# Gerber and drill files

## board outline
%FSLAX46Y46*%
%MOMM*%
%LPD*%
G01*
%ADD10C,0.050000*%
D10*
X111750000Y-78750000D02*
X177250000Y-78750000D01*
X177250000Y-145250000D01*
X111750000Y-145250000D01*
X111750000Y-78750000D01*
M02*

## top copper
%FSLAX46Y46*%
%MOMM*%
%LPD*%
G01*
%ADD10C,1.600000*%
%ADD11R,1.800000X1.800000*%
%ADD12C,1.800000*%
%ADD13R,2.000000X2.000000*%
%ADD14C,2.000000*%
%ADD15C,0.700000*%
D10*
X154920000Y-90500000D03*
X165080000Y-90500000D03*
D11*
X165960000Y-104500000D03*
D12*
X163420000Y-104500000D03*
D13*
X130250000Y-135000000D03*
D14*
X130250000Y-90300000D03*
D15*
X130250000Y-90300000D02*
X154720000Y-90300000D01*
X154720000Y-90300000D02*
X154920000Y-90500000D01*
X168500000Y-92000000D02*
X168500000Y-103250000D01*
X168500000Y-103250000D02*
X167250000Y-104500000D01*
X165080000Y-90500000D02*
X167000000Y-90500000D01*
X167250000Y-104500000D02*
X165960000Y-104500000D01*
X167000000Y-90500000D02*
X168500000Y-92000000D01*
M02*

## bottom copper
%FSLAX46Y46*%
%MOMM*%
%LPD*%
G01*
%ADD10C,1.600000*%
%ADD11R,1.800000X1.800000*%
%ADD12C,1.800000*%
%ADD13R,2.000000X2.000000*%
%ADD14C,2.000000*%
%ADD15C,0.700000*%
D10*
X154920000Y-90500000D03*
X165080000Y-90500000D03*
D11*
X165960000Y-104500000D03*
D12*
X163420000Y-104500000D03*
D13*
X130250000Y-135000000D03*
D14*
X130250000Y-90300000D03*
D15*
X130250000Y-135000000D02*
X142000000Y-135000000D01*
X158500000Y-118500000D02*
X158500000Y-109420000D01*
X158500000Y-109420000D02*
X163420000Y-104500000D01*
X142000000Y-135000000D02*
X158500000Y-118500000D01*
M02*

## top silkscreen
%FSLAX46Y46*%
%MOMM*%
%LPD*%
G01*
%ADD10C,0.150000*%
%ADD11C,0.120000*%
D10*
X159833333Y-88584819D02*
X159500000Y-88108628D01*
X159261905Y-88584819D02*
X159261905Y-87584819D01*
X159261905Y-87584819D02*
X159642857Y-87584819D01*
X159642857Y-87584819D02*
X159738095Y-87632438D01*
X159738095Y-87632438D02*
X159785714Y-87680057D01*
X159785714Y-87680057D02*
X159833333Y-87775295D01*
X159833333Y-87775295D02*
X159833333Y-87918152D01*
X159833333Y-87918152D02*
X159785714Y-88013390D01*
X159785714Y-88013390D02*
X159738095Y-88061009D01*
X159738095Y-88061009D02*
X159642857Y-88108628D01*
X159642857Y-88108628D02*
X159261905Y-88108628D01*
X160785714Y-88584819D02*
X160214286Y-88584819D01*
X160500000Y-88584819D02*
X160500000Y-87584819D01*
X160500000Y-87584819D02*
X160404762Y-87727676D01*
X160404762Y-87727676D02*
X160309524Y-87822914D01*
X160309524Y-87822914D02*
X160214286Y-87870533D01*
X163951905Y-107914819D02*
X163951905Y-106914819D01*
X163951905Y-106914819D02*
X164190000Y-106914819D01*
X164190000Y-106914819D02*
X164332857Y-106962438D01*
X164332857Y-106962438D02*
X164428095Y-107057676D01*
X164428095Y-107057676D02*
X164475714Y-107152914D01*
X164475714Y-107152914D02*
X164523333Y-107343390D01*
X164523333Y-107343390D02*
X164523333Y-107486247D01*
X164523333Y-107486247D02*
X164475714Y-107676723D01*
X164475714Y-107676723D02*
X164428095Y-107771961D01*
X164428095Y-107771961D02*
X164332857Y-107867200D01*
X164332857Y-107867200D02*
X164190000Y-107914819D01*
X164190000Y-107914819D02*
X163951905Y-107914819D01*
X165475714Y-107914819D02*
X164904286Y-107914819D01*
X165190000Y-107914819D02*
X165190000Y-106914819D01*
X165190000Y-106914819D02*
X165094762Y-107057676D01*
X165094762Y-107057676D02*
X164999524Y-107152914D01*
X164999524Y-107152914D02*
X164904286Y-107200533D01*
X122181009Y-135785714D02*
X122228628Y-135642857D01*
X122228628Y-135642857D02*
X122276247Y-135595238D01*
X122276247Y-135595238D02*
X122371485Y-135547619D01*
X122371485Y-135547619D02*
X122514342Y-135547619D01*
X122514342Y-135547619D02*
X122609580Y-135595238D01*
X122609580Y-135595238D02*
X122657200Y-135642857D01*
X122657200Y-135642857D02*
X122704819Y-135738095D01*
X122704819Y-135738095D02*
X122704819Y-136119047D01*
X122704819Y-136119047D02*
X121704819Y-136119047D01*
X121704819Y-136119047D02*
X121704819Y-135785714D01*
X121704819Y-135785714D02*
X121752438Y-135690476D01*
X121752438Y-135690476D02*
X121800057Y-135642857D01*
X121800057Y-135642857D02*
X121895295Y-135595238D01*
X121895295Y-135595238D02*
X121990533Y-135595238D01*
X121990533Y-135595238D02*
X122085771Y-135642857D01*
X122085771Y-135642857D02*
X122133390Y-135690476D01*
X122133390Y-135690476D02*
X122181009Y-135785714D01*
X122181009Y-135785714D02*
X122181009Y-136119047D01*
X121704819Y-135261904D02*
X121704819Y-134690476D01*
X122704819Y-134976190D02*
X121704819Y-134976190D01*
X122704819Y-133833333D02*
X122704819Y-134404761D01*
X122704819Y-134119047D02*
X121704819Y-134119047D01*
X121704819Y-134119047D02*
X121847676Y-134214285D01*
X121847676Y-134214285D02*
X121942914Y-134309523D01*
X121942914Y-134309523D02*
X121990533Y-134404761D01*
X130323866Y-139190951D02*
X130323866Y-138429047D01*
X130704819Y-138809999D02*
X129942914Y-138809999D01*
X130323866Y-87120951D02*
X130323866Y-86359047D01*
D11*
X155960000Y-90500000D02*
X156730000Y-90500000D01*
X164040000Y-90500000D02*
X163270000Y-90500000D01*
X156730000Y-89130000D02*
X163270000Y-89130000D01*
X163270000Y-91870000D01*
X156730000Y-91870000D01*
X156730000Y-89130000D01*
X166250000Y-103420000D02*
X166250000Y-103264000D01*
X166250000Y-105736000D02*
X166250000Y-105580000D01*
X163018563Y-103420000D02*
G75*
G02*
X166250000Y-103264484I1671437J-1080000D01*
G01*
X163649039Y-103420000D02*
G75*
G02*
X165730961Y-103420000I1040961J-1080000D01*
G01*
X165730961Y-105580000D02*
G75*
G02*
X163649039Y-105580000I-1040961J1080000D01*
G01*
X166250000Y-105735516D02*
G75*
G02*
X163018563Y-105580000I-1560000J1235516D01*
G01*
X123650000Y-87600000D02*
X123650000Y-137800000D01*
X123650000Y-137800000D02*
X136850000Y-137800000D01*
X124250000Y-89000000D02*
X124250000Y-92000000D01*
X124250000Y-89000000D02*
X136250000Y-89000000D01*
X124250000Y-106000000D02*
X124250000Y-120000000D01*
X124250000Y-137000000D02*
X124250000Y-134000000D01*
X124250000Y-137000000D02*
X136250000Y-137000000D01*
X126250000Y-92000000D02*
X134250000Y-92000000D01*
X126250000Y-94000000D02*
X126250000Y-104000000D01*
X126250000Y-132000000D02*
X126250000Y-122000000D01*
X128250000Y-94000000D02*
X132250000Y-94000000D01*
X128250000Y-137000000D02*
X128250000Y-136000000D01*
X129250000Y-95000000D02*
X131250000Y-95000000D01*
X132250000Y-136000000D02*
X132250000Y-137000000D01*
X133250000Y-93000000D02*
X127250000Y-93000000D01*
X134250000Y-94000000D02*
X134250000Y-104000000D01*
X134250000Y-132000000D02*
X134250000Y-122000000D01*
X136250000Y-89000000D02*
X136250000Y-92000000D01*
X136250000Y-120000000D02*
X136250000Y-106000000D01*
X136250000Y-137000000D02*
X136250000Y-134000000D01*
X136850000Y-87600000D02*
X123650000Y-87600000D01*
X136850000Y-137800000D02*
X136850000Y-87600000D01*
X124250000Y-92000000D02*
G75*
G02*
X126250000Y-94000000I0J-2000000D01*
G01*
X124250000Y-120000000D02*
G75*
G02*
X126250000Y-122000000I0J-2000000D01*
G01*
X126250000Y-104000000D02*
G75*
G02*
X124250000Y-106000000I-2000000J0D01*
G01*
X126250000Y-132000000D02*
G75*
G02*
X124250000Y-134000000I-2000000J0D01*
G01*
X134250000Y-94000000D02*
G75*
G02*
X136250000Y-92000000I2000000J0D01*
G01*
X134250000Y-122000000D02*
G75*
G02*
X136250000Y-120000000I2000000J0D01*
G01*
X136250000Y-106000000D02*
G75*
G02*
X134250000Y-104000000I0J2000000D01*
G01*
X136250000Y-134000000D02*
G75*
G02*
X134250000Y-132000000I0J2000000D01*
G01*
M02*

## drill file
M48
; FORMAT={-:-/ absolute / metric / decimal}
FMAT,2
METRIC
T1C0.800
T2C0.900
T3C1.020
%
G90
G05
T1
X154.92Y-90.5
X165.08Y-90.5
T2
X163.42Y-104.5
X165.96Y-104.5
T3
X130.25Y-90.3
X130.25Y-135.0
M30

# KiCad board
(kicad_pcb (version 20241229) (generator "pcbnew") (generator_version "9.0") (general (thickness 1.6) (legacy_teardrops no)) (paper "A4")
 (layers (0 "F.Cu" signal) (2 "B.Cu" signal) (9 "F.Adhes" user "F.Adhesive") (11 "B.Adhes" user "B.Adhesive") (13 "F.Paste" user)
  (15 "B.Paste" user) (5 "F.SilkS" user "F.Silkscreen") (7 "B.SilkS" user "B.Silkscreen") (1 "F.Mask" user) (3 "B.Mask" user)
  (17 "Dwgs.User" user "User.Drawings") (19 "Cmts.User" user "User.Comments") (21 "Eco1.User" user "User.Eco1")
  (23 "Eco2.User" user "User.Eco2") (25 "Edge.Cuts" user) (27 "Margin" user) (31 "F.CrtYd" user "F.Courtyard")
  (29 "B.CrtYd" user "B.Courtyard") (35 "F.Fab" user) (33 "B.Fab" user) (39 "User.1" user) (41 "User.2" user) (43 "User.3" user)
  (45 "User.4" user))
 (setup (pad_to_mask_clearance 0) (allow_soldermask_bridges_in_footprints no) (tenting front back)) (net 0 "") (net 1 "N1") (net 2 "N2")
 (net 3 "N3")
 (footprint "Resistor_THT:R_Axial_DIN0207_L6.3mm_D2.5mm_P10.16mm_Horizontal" (layer "F.Cu") (at 154.92 90.5)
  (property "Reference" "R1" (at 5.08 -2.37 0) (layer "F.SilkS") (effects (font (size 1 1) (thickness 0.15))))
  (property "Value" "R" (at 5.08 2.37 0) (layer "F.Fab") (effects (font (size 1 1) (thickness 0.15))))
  (fp_line (start 1.04 0) (end 1.81 0) (stroke (width 0.12) (type solid)) (layer "F.SilkS"))
  (fp_line (start 9.12 0) (end 8.35 0) (stroke (width 0.12) (type solid)) (layer "F.SilkS"))
  (fp_rect (start 1.81 -1.37) (end 8.35 1.37) (stroke (width 0.12) (type solid)) (fill no) (layer "F.SilkS"))
  (pad "1" thru_hole circle (at 0 0) (size 1.6 1.6) (drill 0.8) (layers "*.Cu" "*.Mask") (remove_unused_layers no) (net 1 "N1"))
  (pad "2" thru_hole circle (at 10.16 0) (size 1.6 1.6) (drill 0.8) (layers "*.Cu" "*.Mask") (remove_unused_layers no) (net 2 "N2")))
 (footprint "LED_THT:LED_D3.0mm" (layer "F.Cu") (at 165.96 104.5 180)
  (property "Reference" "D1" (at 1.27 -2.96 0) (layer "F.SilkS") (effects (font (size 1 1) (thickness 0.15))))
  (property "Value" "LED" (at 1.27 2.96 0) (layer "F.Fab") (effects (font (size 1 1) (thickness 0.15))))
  (fp_line (start -0.29 1.08) (end -0.29 1.236) (stroke (width 0.12) (type solid)) (layer "F.SilkS"))
  (fp_line (start -0.29 -1.236) (end -0.29 -1.08) (stroke (width 0.12) (type solid)) (layer "F.SilkS"))
  (fp_arc (start 2.941437 1.08) (mid 1.36566 1.987699) (end -0.29 1.235516) (stroke (width 0.12) (type solid)) (layer "F.SilkS"))
  (fp_arc (start 2.310961 1.08) (mid 1.27 1.5) (end 0.229039 1.08) (stroke (width 0.12) (type solid)) (layer "F.SilkS"))
  (fp_arc (start 0.229039 -1.08) (mid 1.27 -1.5) (end 2.310961 -1.08) (stroke (width 0.12) (type solid)) (layer "F.SilkS"))
  (fp_arc (start -0.29 -1.235516) (mid 1.36566 -1.987699) (end 2.941437 -1.08) (stroke (width 0.12) (type solid)) (layer "F.SilkS"))
  (pad "1" thru_hole rect (at 0 0 180) (size 1.8 1.8) (drill 0.9) (layers "*.Cu" "*.Mask") (remove_unused_layers no) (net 2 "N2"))
  (pad "2" thru_hole circle (at 2.54 0 180) (size 1.8 1.8) (drill 0.9) (layers "*.Cu" "*.Mask") (remove_unused_layers no) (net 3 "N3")))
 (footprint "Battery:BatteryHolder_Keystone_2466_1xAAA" (layer "F.Cu") (at 130.25 135 90)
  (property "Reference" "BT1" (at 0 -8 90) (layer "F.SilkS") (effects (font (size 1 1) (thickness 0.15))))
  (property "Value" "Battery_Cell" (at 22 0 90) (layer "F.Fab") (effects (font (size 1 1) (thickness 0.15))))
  (fp_line (start 47.4 -6.6) (end -2.8 -6.6) (stroke (width 0.12) (type solid)) (layer "F.SilkS"))
  (fp_line (start -2.8 -6.6) (end -2.8 6.6) (stroke (width 0.12) (type solid)) (layer "F.SilkS"))
  (fp_line (start 46 -6) (end 43 -6) (stroke (width 0.12) (type solid)) (layer "F.SilkS"))
  (fp_line (start 46 -6) (end 46 6) (stroke (width 0.12) (type solid)) (layer "F.SilkS"))
  (fp_line (start 29 -6) (end 15 -6) (stroke (width 0.12) (type solid)) (layer "F.SilkS"))
  (fp_line (start -2 -6) (end 1 -6) (stroke (width 0.12) (type solid)) (layer "F.SilkS"))
  (fp_line (start -2 -6) (end -2 6) (stroke (width 0.12) (type solid)) (layer "F.SilkS"))
  (fp_line (start 43 -4) (end 43 4) (stroke (width 0.12) (type solid)) (layer "F.SilkS"))
  (fp_line (start 41 -4) (end 31 -4) (stroke (width 0.12) (type solid)) (layer "F.SilkS"))
  (fp_line (start 3 -4) (end 13 -4) (stroke (width 0.12) (type solid)) (layer "F.SilkS"))
  (fp_line (start 41 -2) (end 41 2) (stroke (width 0.12) (type solid)) (layer "F.SilkS"))
  (fp_line (start -2 -2) (end -1 -2) (stroke (width 0.12) (type solid)) (layer "F.SilkS"))
  (fp_line (start 40 -1) (end 40 1) (stroke (width 0.12) (type solid)) (layer "F.SilkS"))
  (fp_line (start -1 2) (end -2 2) (stroke (width 0.12) (type solid)) (layer "F.SilkS"))
  (fp_line (start 42 3) (end 42 -3) (stroke (width 0.12) (type solid)) (layer "F.SilkS"))
  (fp_line (start 41 4) (end 31 4) (stroke (width 0.12) (type solid)) (layer "F.SilkS"))
  (fp_line (start 3 4) (end 13 4) (stroke (width 0.12) (type solid)) (layer "F.SilkS"))
  (fp_line (start 46 6) (end 43 6) (stroke (width 0.12) (type solid)) (layer "F.SilkS"))
  (fp_line (start 15 6) (end 29 6) (stroke (width 0.12) (type solid)) (layer "F.SilkS"))
  (fp_line (start -2 6) (end 1 6) (stroke (width 0.12) (type solid)) (layer "F.SilkS"))
  (fp_line (start 47.4 6.6) (end 47.4 -6.6) (stroke (width 0.12) (type solid)) (layer "F.SilkS"))
  (fp_line (start -2.8 6.6) (end 47.4 6.6) (stroke (width 0.12) (type solid)) (layer "F.SilkS"))
  (fp_arc (start 43 -6) (mid 42.414214 -4.585786) (end 41 -4) (stroke (width 0.12) (type solid)) (layer "F.SilkS"))
  (fp_arc (start 15 -6) (mid 14.414214 -4.585786) (end 13 -4) (stroke (width 0.12) (type solid)) (layer "F.SilkS"))
  (fp_arc (start 31 -4) (mid 29.585786 -4.585786) (end 29 -6) (stroke (width 0.12) (type solid)) (layer "F.SilkS"))
  (fp_arc (start 3 -4) (mid 1.585786 -4.585786) (end 1 -6) (stroke (width 0.12) (type solid)) (layer "F.SilkS"))
  (fp_arc (start 41 4) (mid 42.414214 4.585786) (end 43 6) (stroke (width 0.12) (type solid)) (layer "F.SilkS"))
  (fp_arc (start 13 4) (mid 14.414214 4.585786) (end 15 6) (stroke (width 0.12) (type solid)) (layer "F.SilkS"))
  (fp_arc (start 29 6) (mid 29.585786 4.585786) (end 31 4) (stroke (width 0.12) (type solid)) (layer "F.SilkS"))
  (fp_arc (start 1 6) (mid 1.585786 4.585786) (end 3 4) (stroke (width 0.12) (type solid)) (layer "F.SilkS"))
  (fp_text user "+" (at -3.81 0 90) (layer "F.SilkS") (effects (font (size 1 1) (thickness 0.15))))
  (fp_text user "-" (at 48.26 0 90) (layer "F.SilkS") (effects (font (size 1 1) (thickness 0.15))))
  (pad "1" thru_hole rect (at 0 0 90) (size 2 2) (drill 1.02) (layers "*.Cu" "*.Mask") (remove_unused_layers no) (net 3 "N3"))
  (pad "2" thru_hole circle (at 44.7 0 90) (size 2 2) (drill 1.02) (layers "*.Cu" "*.Mask") (remove_unused_layers no) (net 1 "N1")))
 (gr_rect (start 111.75 78.75) (end 177.25 145.25) (stroke (width 0.05) (type default)) (fill no) (layer "Edge.Cuts"))
 (segment (start 130.25 90.3) (end 154.72 90.3) (width 0.7) (layer "F.Cu") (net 1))
 (segment (start 154.72 90.3) (end 154.92 90.5) (width 0.7) (layer "F.Cu") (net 1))
 (segment (start 168.5 92) (end 168.5 103.25) (width 0.7) (layer "F.Cu") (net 2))
 (segment (start 168.5 103.25) (end 167.25 104.5) (width 0.7) (layer "F.Cu") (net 2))
 (segment (start 165.08 90.5) (end 167 90.5) (width 0.7) (layer "F.Cu") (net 2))
 (segment (start 167.25 104.5) (end 165.96 104.5) (width 0.7) (layer "F.Cu") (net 2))
 (segment (start 167 90.5) (end 168.5 92) (width 0.7) (layer "F.Cu") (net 2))
 (segment (start 130.25 135) (end 142 135) (width 0.7) (layer "B.Cu") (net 3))
 (segment (start 158.5 118.5) (end 158.5 109.42) (width 0.7) (layer "B.Cu") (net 3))
 (segment (start 158.5 109.42) (end 163.42 104.5) (width 0.7) (layer "B.Cu") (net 3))
 (segment (start 142 135) (end 158.5 118.5) (width 0.7) (layer "B.Cu") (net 3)))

